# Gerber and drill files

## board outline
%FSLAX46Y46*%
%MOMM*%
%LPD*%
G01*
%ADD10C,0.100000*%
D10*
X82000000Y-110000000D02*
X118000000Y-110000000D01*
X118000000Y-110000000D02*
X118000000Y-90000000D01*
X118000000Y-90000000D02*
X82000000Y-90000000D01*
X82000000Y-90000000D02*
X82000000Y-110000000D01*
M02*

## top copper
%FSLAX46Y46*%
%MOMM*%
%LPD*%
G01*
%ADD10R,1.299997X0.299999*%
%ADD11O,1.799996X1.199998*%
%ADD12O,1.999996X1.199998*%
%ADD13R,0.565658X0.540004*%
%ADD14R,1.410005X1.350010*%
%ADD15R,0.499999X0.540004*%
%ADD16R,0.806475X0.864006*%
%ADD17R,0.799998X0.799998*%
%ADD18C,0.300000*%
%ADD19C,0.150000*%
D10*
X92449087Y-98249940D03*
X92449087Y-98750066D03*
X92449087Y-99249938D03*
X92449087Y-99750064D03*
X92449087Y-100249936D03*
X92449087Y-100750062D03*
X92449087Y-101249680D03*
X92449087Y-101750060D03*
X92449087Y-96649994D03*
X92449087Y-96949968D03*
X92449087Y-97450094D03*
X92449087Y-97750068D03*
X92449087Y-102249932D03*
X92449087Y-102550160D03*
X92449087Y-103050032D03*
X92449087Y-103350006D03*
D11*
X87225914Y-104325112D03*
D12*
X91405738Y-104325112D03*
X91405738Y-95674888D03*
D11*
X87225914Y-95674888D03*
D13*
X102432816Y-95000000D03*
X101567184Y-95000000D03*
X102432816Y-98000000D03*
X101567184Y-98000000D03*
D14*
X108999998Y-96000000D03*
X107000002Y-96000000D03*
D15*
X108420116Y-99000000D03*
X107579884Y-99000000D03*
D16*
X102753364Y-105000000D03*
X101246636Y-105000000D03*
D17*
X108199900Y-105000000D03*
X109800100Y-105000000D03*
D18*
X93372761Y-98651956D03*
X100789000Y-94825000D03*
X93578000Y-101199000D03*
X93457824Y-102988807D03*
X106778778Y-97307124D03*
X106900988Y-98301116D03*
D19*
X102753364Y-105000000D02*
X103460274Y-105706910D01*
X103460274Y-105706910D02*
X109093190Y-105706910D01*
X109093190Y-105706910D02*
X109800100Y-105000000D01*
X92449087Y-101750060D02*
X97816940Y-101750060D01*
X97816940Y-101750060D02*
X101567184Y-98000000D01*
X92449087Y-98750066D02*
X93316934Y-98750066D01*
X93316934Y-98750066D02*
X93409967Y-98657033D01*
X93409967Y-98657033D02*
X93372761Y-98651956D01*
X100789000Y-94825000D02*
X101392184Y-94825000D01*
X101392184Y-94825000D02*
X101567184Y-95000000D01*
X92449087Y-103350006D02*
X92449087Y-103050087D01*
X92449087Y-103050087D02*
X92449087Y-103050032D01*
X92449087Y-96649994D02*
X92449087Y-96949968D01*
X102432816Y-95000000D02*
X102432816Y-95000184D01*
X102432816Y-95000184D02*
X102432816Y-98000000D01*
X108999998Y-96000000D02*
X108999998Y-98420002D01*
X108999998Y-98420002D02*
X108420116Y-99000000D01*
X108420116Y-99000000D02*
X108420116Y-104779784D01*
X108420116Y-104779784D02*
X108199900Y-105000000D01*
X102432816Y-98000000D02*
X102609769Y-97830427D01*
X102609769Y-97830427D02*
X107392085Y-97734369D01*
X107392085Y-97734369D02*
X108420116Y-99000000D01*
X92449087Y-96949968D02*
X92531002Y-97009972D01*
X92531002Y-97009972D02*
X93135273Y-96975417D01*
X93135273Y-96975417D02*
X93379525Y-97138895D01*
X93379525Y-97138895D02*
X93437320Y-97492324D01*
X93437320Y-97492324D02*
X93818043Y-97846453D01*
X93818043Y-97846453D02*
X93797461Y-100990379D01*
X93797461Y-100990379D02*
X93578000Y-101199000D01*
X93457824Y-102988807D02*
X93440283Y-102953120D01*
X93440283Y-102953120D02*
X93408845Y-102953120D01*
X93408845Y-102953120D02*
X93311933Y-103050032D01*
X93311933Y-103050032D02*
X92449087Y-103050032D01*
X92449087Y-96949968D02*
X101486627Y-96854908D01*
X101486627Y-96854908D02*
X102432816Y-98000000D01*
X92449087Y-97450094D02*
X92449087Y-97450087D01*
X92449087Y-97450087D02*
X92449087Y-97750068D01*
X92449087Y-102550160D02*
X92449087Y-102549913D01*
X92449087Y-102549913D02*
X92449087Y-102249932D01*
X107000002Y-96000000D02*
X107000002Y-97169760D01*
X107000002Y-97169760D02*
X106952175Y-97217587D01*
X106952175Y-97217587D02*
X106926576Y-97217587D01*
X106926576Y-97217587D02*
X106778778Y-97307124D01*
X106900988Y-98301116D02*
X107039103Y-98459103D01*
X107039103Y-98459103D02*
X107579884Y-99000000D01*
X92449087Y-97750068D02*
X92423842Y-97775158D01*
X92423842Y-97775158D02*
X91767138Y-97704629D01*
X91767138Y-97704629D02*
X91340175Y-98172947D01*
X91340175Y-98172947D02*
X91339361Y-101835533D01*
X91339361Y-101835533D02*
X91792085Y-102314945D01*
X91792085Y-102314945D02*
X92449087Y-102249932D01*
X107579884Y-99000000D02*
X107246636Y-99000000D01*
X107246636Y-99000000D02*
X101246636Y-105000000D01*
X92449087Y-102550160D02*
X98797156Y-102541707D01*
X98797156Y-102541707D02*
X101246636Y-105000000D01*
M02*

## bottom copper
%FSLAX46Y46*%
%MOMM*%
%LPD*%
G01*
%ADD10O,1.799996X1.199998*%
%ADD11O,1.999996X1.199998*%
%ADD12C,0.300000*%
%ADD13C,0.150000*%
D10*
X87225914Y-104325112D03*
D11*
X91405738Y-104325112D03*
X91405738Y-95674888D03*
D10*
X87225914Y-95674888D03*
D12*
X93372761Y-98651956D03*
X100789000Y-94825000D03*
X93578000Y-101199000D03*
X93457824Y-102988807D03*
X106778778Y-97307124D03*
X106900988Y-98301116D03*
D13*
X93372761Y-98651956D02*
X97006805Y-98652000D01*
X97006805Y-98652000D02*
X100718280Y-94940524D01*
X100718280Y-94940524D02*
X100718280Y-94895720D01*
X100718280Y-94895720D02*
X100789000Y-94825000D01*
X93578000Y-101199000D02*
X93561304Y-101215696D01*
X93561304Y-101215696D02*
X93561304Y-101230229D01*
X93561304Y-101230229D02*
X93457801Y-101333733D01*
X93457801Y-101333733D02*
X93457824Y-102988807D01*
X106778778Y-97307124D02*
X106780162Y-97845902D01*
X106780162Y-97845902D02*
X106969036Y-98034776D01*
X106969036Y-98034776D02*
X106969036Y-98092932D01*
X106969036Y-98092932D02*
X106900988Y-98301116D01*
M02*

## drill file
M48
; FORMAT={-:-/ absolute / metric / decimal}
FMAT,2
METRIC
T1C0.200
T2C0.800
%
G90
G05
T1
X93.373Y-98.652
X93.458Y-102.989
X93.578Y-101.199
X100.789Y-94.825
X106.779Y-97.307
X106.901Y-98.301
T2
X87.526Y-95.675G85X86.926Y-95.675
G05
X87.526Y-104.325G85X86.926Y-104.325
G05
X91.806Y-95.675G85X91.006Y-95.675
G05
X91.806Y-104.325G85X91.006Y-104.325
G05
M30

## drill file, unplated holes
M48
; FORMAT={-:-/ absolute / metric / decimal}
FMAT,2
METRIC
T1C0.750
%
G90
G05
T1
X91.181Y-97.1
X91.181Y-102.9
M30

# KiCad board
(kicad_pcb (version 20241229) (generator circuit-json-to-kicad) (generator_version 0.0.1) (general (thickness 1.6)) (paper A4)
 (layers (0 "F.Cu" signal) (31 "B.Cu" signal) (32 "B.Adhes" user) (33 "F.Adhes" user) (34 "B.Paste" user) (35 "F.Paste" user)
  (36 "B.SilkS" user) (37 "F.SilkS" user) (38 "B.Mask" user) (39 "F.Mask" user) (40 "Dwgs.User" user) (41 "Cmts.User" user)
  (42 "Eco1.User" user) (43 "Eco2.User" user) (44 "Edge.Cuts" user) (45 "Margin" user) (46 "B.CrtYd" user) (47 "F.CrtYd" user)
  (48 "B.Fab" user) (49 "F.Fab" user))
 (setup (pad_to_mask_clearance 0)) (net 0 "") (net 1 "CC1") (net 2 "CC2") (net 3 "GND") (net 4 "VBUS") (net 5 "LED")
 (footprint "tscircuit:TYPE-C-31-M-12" (layer F.Cu) (at 90 100 270)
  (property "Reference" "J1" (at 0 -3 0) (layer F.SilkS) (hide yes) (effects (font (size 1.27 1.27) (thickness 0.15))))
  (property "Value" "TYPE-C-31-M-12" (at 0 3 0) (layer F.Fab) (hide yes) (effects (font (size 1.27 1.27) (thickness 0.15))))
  (pad "5" smd rect (at -1.7500600000000766 -2.449087049999889 0) (size 1.2999973999999999 0.29999939999999997) (layers F.Cu F.Mask))
  (pad "6" smd rect (at -1.24993399999994 -2.449087049999889 0) (size 1.2999973999999999 0.29999939999999997) (layers F.Cu F.Mask)
   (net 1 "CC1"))
  (pad "7" smd rect (at -0.7500619999999578 -2.449087049999889 0) (size 1.2999973999999999 0.29999939999999997) (layers F.Cu F.Mask))
  (pad "8" smd rect (at -0.2499359999999348 -2.449087049999889 0) (size 1.2999973999999999 0.29999939999999997) (layers F.Cu F.Mask))
  (pad "9" smd rect (at 0.24993599999993363 -2.449087049999889 0) (size 1.2999973999999999 0.29999939999999997) (layers F.Cu F.Mask))
  (pad "10" smd rect (at 0.7500619999999565 -2.449087049999889 0) (size 1.2999973999999999 0.29999939999999997) (layers F.Cu F.Mask))
  (pad "11" smd rect (at 1.2496799999998978 -2.449087049999889 0) (size 1.2999973999999999 0.29999939999999997) (layers F.Cu F.Mask))
  (pad "12" smd rect (at 1.7500600000000752 -2.449087049999889 0) (size 1.2999973999999999 0.29999939999999997) (layers F.Cu F.Mask)
   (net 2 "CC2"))
  (pad "1" smd rect (at -3.350006000000008 -2.4490870499998882 0) (size 1.2999973999999999 0.29999939999999997) (layers F.Cu F.Mask)
   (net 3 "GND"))
  (pad "2" smd rect (at -3.050031999999988 -2.4490870499998882 0) (size 1.2999973999999999 0.29999939999999997) (layers F.Cu F.Mask)
   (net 3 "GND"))
  (pad "3" smd rect (at -2.549905999999965 -2.4490870499998882 0) (size 1.2999973999999999 0.29999939999999997) (layers F.Cu F.Mask)
   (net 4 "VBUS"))
  (pad "4" smd rect (at -2.2499320000000584 -2.449087049999889 0) (size 1.2999973999999999 0.29999939999999997) (layers F.Cu F.Mask)
   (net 4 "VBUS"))
  (pad "14" smd rect (at 2.2499320000000576 -2.449087049999889 0) (size 1.2999973999999999 0.29999939999999997) (layers F.Cu F.Mask)
   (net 4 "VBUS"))
  (pad "13" smd rect (at 2.550160000000005 -2.44908704999989 0) (size 1.2999973999999999 0.29999939999999997) (layers F.Cu F.Mask)
   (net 4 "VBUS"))
  (pad "16" smd rect (at 3.0500320000001007 -2.44908704999989 0) (size 1.2999973999999999 0.29999939999999997) (layers F.Cu F.Mask)
   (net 3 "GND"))
  (pad "15" smd rect (at 3.350006000000007 -2.44908704999989 0) (size 1.2999973999999999 0.29999939999999997) (layers F.Cu F.Mask)
   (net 3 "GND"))
  (pad "" smd roundrect (at 4.325111999999991 2.7740863499999477 270) (size 1.1999975999999999 1.7999964) (layers F.Paste)
   (roundrect_rratio 0.5))
  (pad "" smd roundrect (at 4.325111999999991 2.7740863499999477 270) (size 1.1999975999999999 1.7999964) (layers B.Paste)
   (roundrect_rratio 0.5))
  (pad "" smd roundrect (at 4.32511199999999 -1.4057376499998782 270) (size 1.1999975999999999 1.9999959999999999) (layers F.Paste)
   (roundrect_rratio 0.5))
  (pad "" smd roundrect (at 4.32511199999999 -1.4057376499998782 270) (size 1.1999975999999999 1.9999959999999999) (layers B.Paste)
   (roundrect_rratio 0.5))
  (pad "" smd roundrect (at -4.32511199999999 -1.4057376499998782 270) (size 1.1999975999999999 1.9999959999999999) (layers F.Paste)
   (roundrect_rratio 0.5))
  (pad "" smd roundrect (at -4.32511199999999 -1.4057376499998782 270) (size 1.1999975999999999 1.9999959999999999) (layers B.Paste)
   (roundrect_rratio 0.5))
  (pad "" smd roundrect (at -4.325111999999989 2.7740863499999477 270) (size 1.1999975999999999 1.7999964) (layers F.Paste)
   (roundrect_rratio 0.5))
  (pad "" smd roundrect (at -4.325111999999989 2.7740863499999477 270) (size 1.1999975999999999 1.7999964) (layers B.Paste)
   (roundrect_rratio 0.5))
  (pad "" smd rect (at -1.7500600000000766 -2.449087049999889 0) (size 0.9099981799999999 0.20999957999999996) (layers F.Paste))
  (pad "" smd rect (at -1.24993399999994 -2.449087049999889 0) (size 0.9099981799999999 0.20999957999999996) (layers F.Paste))
  (pad "" smd rect (at -0.7500619999999578 -2.449087049999889 0) (size 0.9099981799999999 0.20999957999999996) (layers F.Paste))
  (pad "" smd rect (at -0.2499359999999348 -2.449087049999889 0) (size 0.9099981799999999 0.20999957999999996) (layers F.Paste))
  (pad "" smd rect (at 0.24993599999993363 -2.449087049999889 0) (size 0.9099981799999999 0.20999957999999996) (layers F.Paste))
  (pad "" smd rect (at 0.7500619999999565 -2.449087049999889 0) (size 0.9099981799999999 0.20999957999999996) (layers F.Paste))
  (pad "" smd rect (at 1.2496799999998978 -2.449087049999889 0) (size 0.9099981799999999 0.20999957999999996) (layers F.Paste))
  (pad "" smd rect (at 1.7500600000000752 -2.449087049999889 0) (size 0.9099981799999999 0.20999957999999996) (layers F.Paste))
  (pad "" smd rect (at -3.350006000000008 -2.4490870499998882 0) (size 0.9099981799999999 0.20999957999999996) (layers F.Paste))
  (pad "" smd rect (at -3.050031999999988 -2.4490870499998882 0) (size 0.9099981799999999 0.20999957999999996) (layers F.Paste))
  (pad "" smd rect (at -2.549905999999965 -2.4490870499998882 0) (size 0.9099981799999999 0.20999957999999996) (layers F.Paste))
  (pad "" smd rect (at -2.2499320000000584 -2.449087049999889 0) (size 0.9099981799999999 0.20999957999999996) (layers F.Paste))
  (pad "" smd rect (at 2.2499320000000576 -2.449087049999889 0) (size 0.9099981799999999 0.20999957999999996) (layers F.Paste))
  (pad "" smd rect (at 2.550160000000005 -2.44908704999989 0) (size 0.9099981799999999 0.20999957999999996) (layers F.Paste))
  (pad "" smd rect (at 3.0500320000001007 -2.44908704999989 0) (size 0.9099981799999999 0.20999957999999996) (layers F.Paste))
  (pad "" smd rect (at 3.350006000000007 -2.44908704999989 0) (size 0.9099981799999999 0.20999957999999996) (layers F.Paste))
  (pad "17" thru_hole oval (at 4.325111999999991 2.774086349999947 270) (size 1.1999975999999999 1.7999964)
   (drill oval 0.7999983999999999 1.3999972) (layers *.Cu *.Mask))
  (pad "18" thru_hole oval (at 4.32511199999999 -1.405737649999879 270) (size 1.1999975999999999 1.9999959999999999)
   (drill oval 0.7999983999999999 1.5999968) (layers *.Cu *.Mask))
  (pad "19" thru_hole oval (at -4.32511199999999 -1.4057376499998773 270) (size 1.1999975999999999 1.9999959999999999)
   (drill oval 0.7999983999999999 1.5999968) (layers *.Cu *.Mask))
  (pad "20" thru_hole oval (at -4.325111999999989 2.7740863499999486 270) (size 1.1999975999999999 1.7999964)
   (drill oval 0.7999983999999999 1.3999972) (layers *.Cu *.Mask))
  (pad "" np_thru_hole circle (at -2.8999180000000706 -1.1806110499999245 0) (size 0.7500111999999999 0.7500111999999999)
   (drill 0.7500111999999999) (layers *.Cu *.Mask))
  (pad "" np_thru_hole circle (at 2.8999180000000706 -1.1806110499999254 0) (size 0.7500111999999999 0.7500111999999999)
   (drill 0.7500111999999999) (layers *.Cu *.Mask)))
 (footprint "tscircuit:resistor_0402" (layer F.Cu) (at 102 95 0)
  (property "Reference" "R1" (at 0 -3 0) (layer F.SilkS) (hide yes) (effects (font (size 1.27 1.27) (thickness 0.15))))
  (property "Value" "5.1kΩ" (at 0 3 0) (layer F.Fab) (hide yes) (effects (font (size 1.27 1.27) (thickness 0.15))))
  (pad "2" smd rect (at 0.43281600000000253 0 0) (size 0.565658 0.5400039999999999) (layers F.Cu F.Mask) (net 3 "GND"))
  (pad "1" smd rect (at -0.4328160000001162 0 0) (size 0.565658 0.5400039999999999) (layers F.Cu F.Mask) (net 1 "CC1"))
  (pad "" smd rect (at 0.43281600000000253 0 0) (size 0.3959606 0.3780027999999999) (layers F.Paste))
  (pad "" smd rect (at -0.4328160000001162 0 0) (size 0.3959606 0.3780027999999999) (layers F.Paste)))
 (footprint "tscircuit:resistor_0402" (layer F.Cu) (at 102 98 0)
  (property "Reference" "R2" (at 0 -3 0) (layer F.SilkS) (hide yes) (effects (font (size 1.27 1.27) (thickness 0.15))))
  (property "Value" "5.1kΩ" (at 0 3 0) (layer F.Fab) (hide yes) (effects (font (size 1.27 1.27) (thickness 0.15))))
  (pad "2" smd rect (at 0.43281600000000253 0 0) (size 0.565658 0.5400039999999999) (layers F.Cu F.Mask) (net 3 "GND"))
  (pad "1" smd rect (at -0.4328160000001162 0 0) (size 0.565658 0.5400039999999999) (layers F.Cu F.Mask) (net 2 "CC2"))
  (pad "" smd rect (at 0.43281600000000253 0 0) (size 0.3959606 0.3780027999999999) (layers F.Paste))
  (pad "" smd rect (at -0.4328160000001162 0 0) (size 0.3959606 0.3780027999999999) (layers F.Paste)))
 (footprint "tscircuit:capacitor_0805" (layer F.Cu) (at 108 96 0)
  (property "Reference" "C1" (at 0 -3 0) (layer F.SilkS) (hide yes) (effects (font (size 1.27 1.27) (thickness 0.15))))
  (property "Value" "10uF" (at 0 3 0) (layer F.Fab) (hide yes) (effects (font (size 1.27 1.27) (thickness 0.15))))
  (pad "2" smd rect (at 0.9999979999998914 0 0) (size 1.4100048 1.3500100000000002) (layers F.Cu F.Mask) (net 3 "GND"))
  (pad "1" smd rect (at -0.9999979999998914 0 0) (size 1.4100048 1.3500100000000002) (layers F.Cu F.Mask) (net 4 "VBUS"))
  (pad "" smd rect (at 0.9999979999998914 0 0) (size 0.98700336 0.945007) (layers F.Paste))
  (pad "" smd rect (at -0.9999979999998914 0 0) (size 0.98700336 0.945007) (layers F.Paste)))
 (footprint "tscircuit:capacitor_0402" (layer F.Cu) (at 108 99 0)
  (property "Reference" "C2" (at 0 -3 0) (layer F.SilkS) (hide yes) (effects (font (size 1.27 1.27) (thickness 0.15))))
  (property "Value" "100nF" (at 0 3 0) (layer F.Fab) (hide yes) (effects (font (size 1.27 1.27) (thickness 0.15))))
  (pad "2" smd rect (at 0.42011600000000726 0 0) (size 0.49999899999999997 0.5400039999999999) (layers F.Cu F.Mask) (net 3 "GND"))
  (pad "1" smd rect (at -0.42011600000000726 0 0) (size 0.49999899999999997 0.5400039999999999) (layers F.Cu F.Mask) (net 4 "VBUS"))
  (pad "" smd rect (at 0.42011600000000726 0 0) (size 0.34999929999999996 0.3780027999999999) (layers F.Paste))
  (pad "" smd rect (at -0.42011600000000726 0 0) (size 0.34999929999999996 0.3780027999999999) (layers F.Paste)))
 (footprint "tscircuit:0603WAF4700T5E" (layer F.Cu) (at 102 105 0)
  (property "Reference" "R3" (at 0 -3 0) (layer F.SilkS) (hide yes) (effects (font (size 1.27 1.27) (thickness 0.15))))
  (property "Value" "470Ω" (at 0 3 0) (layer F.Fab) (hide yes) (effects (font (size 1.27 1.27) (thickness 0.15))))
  (pad "2" smd rect (at 0.7533639999998059 0 0) (size 0.8064754 0.8640064000000001) (layers F.Cu F.Mask) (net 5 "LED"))
  (pad "1" smd rect (at -0.7533639999999195 0 0) (size 0.8064754 0.8640064000000001) (layers F.Cu F.Mask) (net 4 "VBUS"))
  (pad "" smd rect (at 0.7533639999998059 0 0) (size 0.56453278 0.60480448) (layers F.Paste))
  (pad "" smd rect (at -0.7533639999999195 0 0) (size 0.56453278 0.60480448) (layers F.Paste)))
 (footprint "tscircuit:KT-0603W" (layer F.Cu) (at 109 105 0)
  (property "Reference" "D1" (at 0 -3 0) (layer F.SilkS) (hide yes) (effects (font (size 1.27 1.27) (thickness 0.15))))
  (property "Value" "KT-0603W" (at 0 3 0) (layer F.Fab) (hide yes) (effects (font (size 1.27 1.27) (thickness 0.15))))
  (pad "2" smd rect (at -0.8000999999999294 0 0) (size 0.7999983999999999 0.7999983999999999) (layers F.Cu F.Mask) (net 3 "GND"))
  (pad "1" smd rect (at 0.8001000000000431 0 0) (size 0.7999983999999999 0.7999983999999999) (layers F.Cu F.Mask) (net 5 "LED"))
  (pad "" smd rect (at -0.8000999999999294 0 0) (size 0.5599988799999999 0.5599988799999999) (layers F.Paste))
  (pad "" smd rect (at 0.8001000000000431 0 0) (size 0.5599988799999999 0.5599988799999999) (layers F.Paste)))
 (segment (start 102.7533639999998 105) (end 103.46027418090058 105.70691018090078) (width 0.15) (layer F.Cu) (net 5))
 (segment (start 103.46027418090058 105.70691018090078) (end 109.09318981909927 105.70691018090078) (width 0.15) (layer F.Cu) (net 5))
 (segment (start 109.09318981909927 105.70691018090078) (end 109.80010000000004 105) (width 0.15) (layer F.Cu) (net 5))
 (segment (start 92.44908704999989 101.75006000000008) (end 97.81693999999993 101.75006000000008) (width 0.15) (layer F.Cu) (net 2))
 (segment (start 97.81693999999993 101.75006000000008) (end 101.56718399999988 98) (width 0.15) (layer F.Cu) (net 2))
 (segment (start 92.44908704999989 98.75006600000006) (end 93.31693399999995 98.75006600000006) (width 0.15) (layer F.Cu) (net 1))
 (segment (start 93.31693399999995 98.75006600000006) (end 93.40996694834767 98.65703305165232) (width 0.15) (layer F.Cu) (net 1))
 (segment (start 93.40996694834767 98.65703305165232) (end 93.37276085278589 98.65195569042825) (width 0.15) (layer F.Cu) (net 1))
 (segment (start 93.37276085278589 98.65195569042825) (end 97.00680465647108 98.652) (width 0.15) (layer B.Cu) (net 1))
 (segment (start 97.00680465647108 98.652) (end 100.71828030536405 94.94052435110703) (width 0.15) (layer B.Cu) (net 1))
 (segment (start 100.71828030536405 94.94052435110703) (end 100.71828030536405 94.89571969463596) (width 0.15) (layer B.Cu) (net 1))
 (segment (start 100.71828030536405 94.89571969463596) (end 100.789 94.825) (width 0.15) (layer B.Cu) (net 1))
 (segment (start 100.789 94.825) (end 101.39218399999989 94.825) (width 0.15) (layer F.Cu) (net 1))
 (segment (start 101.39218399999989 94.825) (end 101.56718399999988 95) (width 0.15) (layer F.Cu) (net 1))
 (segment (start 92.44908704999989 103.35000600000001) (end 92.44908704999989 103.05008704999989) (width 0.15) (layer F.Cu) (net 3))
 (segment (start 92.44908704999989 103.05008704999989) (end 92.44908704999989 103.0500320000001) (width 0.15) (layer F.Cu) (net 3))
 (segment (start 92.44908704999989 96.64999399999999) (end 92.44908704999989 96.94996800000001) (width 0.15) (layer F.Cu) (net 3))
 (segment (start 102.432816 95) (end 102.432816 95.00018399999999) (width 0.15) (layer F.Cu) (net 3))
 (segment (start 102.432816 95.00018399999999) (end 102.432816 98) (width 0.15) (layer F.Cu) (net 3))
 (segment (start 108.99999799999989 96) (end 108.99999799999989 98.42000200000011) (width 0.15) (layer F.Cu) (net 3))
 (segment (start 108.99999799999989 98.42000200000011) (end 108.42011600000001 99) (width 0.15) (layer F.Cu) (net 3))
 (segment (start 108.42011600000001 99) (end 108.42011600000001 104.77978400000006) (width 0.15) (layer F.Cu) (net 3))
 (segment (start 108.42011600000001 104.77978400000006) (end 108.19990000000007 105) (width 0.15) (layer F.Cu) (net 3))
 (segment (start 102.432816 98) (end 102.6097687741326 97.83042654985954) (width 0.15) (layer F.Cu) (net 3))
 (segment (start 102.6097687741326 97.83042654985954) (end 107.39208477508505 97.73436864948413) (width 0.15) (layer F.Cu) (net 3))
 (segment (start 107.39208477508505 97.73436864948413) (end 108.42011600000001 99) (width 0.15) (layer F.Cu) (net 3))
 (segment (start 92.44908704999989 96.94996800000001) (end 92.53100207613589 97.00997243178794) (width 0.15) (layer F.Cu) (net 3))
 (segment (start 92.53100207613589 97.00997243178794) (end 93.13527277548843 96.97541700786259) (width 0.15) (layer F.Cu) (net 3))
 (segment (start 93.13527277548843 96.97541700786259) (end 93.37952517299357 97.13889481872864) (width 0.15) (layer F.Cu) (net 3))
 (segment (start 93.37952517299357 97.13889481872864) (end 93.43732045464824 97.49232386105668) (width 0.15) (layer F.Cu) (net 3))
 (segment (start 93.43732045464824 97.49232386105668) (end 93.81804270431249 97.84645337660929) (width 0.15) (layer F.Cu) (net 3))
 (segment (start 93.81804270431249 97.84645337660929) (end 93.79746121192701 100.9903787865805) (width 0.15) (layer F.Cu) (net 3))
 (segment (start 93.79746121192701 100.9903787865805) (end 93.578 101.199) (width 0.15) (layer F.Cu) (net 3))
 (segment (start 93.578 101.199) (end 93.56130438446648 101.21569561553352) (width 0.15) (layer B.Cu) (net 3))
 (segment (start 93.56130438446648 101.21569561553352) (end 93.56130438446648 101.23022929295647) (width 0.15) (layer B.Cu) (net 3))
 (segment (start 93.56130438446648 101.23022929295647) (end 93.45780069381489 101.33373298360806) (width 0.15) (layer B.Cu) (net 3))
 (segment (start 93.45780069381489 101.33373298360806) (end 93.45782390664056 102.98880739026725) (width 0.15) (layer B.Cu) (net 3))
 (segment (start 93.45782390664056 102.98880739026725) (end 93.44028304706794 102.9531196203537) (width 0.15) (layer F.Cu) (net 3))
 (segment (start 93.44028304706794 102.9531196203537) (end 93.40884514376495 102.9531196203537) (width 0.15) (layer F.Cu) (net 3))
 (segment (start 93.40884514376495 102.9531196203537) (end 93.31193276411855 103.0500320000001) (width 0.15) (layer F.Cu) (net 3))
 (segment (start 93.31193276411855 103.0500320000001) (end 92.44908704999989 103.0500320000001) (width 0.15) (layer F.Cu) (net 3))
 (segment (start 92.44908704999989 96.94996800000001) (end 101.48662713053767 96.85490803018594) (width 0.15) (layer F.Cu) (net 3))
 (segment (start 101.48662713053767 96.85490803018594) (end 102.432816 98) (width 0.15) (layer F.Cu) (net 3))
 (segment (start 92.44908704999989 97.45009400000004) (end 92.44908704999989 97.4500870499999) (width 0.15) (layer F.Cu) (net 4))
 (segment (start 92.44908704999989 97.4500870499999) (end 92.44908704999989 97.75006799999994) (width 0.15) (layer F.Cu) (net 4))
 (segment (start 92.44908704999989 102.55016) (end 92.44908704999989 102.5499129500001) (width 0.15) (layer F.Cu) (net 4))
 (segment (start 92.44908704999989 102.5499129500001) (end 92.44908704999989 102.24993200000006) (width 0.15) (layer F.Cu) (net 4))
 (segment (start 107.00000200000011 96) (end 107.00000200000011 97.1697598967502) (width 0.15) (layer F.Cu) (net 4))
 (segment (start 107.00000200000011 97.1697598967502) (end 106.95217527479988 97.21758662195043) (width 0.15) (layer F.Cu) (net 4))
 (segment (start 106.95217527479988 97.21758662195043) (end 106.92657553531514 97.21758662195043) (width 0.15) (layer F.Cu) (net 4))
 (segment (start 106.92657553531514 97.21758662195043) (end 106.77877844696536 97.3071235694304) (width 0.15) (layer F.Cu) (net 4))
 (segment (start 106.77877844696536 97.3071235694304) (end 106.78016215726556 97.84590189939782) (width 0.15) (layer B.Cu) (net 4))
 (segment (start 106.78016215726556 97.84590189939782) (end 106.96903578095319 98.03477552308543) (width 0.15) (layer B.Cu) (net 4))
 (segment (start 106.96903578095319 98.03477552308543) (end 106.96903578095319 98.09293248003561) (width 0.15) (layer B.Cu) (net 4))
 (segment (start 106.96903578095319 98.09293248003561) (end 106.90098771737058 98.30111558354697) (width 0.15) (layer B.Cu) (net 4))
 (segment (start 106.90098771737058 98.30111558354697) (end 107.03910330091756 98.45910330091756) (width 0.15) (layer F.Cu) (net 4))
 (segment (start 107.03910330091756 98.45910330091756) (end 107.57988399999999 99) (width 0.15) (layer F.Cu) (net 4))
 (segment (start 92.44908704999989 97.75006799999994) (end 92.42384156501494 97.77515843498506) (width 0.15) (layer F.Cu) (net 4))
 (segment (start 92.42384156501494 97.77515843498506) (end 91.76713763144994 97.70462897169368) (width 0.15) (layer F.Cu) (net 4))
 (segment (start 91.76713763144994 97.70462897169368) (end 91.34017483774099 98.17294672915985) (width 0.15) (layer F.Cu) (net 4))
 (segment (start 91.34017483774099 98.17294672915985) (end 91.33936110234858 101.83553289651994) (width 0.15) (layer F.Cu) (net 4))
 (segment (start 91.33936110234858 101.83553289651994) (end 91.79208468073189 102.31494479918398) (width 0.15) (layer F.Cu) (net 4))
 (segment (start 91.79208468073189 102.31494479918398) (end 92.44908704999989 102.24993200000006) (width 0.15) (layer F.Cu) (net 4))
 (segment (start 107.57988399999999 99) (end 107.24663600000008 99) (width 0.15) (layer F.Cu) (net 4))
 (segment (start 107.24663600000008 99) (end 101.24663600000008 105) (width 0.15) (layer F.Cu) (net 4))
 (segment (start 92.44908704999989 102.55016) (end 98.797156312924 102.54170714370545) (width 0.15) (layer F.Cu) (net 4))
 (segment (start 98.797156312924 102.54170714370545) (end 101.24663600000008 105) (width 0.15) (layer F.Cu) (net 4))
 (gr_line (start 82 110) (end 118 110) (width 0.1) (layer Edge.Cuts))
 (gr_line (start 118 110) (end 118 90) (width 0.1) (layer Edge.Cuts))
 (gr_line (start 118 90) (end 82 90) (width 0.1) (layer Edge.Cuts))
 (gr_line (start 82 90) (end 82 110) (width 0.1) (layer Edge.Cuts))
 (via (at 93.37276085278589 98.65195569042825) (size 0.3) (drill 0.2) (layers F.Cu B.Cu) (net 1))
 (via (at 100.789 94.825) (size 0.3) (drill 0.2) (layers F.Cu B.Cu) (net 1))
 (via (at 93.578 101.199) (size 0.3) (drill 0.2) (layers F.Cu B.Cu) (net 3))
 (via (at 93.45782390664056 102.98880739026725) (size 0.3) (drill 0.2) (layers F.Cu B.Cu) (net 3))
 (via (at 106.77877844696536 97.3071235694304) (size 0.3) (drill 0.2) (layers F.Cu B.Cu) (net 4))
 (via (at 106.90098771737058 98.30111558354697) (size 0.3) (drill 0.2) (layers F.Cu B.Cu) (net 4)))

